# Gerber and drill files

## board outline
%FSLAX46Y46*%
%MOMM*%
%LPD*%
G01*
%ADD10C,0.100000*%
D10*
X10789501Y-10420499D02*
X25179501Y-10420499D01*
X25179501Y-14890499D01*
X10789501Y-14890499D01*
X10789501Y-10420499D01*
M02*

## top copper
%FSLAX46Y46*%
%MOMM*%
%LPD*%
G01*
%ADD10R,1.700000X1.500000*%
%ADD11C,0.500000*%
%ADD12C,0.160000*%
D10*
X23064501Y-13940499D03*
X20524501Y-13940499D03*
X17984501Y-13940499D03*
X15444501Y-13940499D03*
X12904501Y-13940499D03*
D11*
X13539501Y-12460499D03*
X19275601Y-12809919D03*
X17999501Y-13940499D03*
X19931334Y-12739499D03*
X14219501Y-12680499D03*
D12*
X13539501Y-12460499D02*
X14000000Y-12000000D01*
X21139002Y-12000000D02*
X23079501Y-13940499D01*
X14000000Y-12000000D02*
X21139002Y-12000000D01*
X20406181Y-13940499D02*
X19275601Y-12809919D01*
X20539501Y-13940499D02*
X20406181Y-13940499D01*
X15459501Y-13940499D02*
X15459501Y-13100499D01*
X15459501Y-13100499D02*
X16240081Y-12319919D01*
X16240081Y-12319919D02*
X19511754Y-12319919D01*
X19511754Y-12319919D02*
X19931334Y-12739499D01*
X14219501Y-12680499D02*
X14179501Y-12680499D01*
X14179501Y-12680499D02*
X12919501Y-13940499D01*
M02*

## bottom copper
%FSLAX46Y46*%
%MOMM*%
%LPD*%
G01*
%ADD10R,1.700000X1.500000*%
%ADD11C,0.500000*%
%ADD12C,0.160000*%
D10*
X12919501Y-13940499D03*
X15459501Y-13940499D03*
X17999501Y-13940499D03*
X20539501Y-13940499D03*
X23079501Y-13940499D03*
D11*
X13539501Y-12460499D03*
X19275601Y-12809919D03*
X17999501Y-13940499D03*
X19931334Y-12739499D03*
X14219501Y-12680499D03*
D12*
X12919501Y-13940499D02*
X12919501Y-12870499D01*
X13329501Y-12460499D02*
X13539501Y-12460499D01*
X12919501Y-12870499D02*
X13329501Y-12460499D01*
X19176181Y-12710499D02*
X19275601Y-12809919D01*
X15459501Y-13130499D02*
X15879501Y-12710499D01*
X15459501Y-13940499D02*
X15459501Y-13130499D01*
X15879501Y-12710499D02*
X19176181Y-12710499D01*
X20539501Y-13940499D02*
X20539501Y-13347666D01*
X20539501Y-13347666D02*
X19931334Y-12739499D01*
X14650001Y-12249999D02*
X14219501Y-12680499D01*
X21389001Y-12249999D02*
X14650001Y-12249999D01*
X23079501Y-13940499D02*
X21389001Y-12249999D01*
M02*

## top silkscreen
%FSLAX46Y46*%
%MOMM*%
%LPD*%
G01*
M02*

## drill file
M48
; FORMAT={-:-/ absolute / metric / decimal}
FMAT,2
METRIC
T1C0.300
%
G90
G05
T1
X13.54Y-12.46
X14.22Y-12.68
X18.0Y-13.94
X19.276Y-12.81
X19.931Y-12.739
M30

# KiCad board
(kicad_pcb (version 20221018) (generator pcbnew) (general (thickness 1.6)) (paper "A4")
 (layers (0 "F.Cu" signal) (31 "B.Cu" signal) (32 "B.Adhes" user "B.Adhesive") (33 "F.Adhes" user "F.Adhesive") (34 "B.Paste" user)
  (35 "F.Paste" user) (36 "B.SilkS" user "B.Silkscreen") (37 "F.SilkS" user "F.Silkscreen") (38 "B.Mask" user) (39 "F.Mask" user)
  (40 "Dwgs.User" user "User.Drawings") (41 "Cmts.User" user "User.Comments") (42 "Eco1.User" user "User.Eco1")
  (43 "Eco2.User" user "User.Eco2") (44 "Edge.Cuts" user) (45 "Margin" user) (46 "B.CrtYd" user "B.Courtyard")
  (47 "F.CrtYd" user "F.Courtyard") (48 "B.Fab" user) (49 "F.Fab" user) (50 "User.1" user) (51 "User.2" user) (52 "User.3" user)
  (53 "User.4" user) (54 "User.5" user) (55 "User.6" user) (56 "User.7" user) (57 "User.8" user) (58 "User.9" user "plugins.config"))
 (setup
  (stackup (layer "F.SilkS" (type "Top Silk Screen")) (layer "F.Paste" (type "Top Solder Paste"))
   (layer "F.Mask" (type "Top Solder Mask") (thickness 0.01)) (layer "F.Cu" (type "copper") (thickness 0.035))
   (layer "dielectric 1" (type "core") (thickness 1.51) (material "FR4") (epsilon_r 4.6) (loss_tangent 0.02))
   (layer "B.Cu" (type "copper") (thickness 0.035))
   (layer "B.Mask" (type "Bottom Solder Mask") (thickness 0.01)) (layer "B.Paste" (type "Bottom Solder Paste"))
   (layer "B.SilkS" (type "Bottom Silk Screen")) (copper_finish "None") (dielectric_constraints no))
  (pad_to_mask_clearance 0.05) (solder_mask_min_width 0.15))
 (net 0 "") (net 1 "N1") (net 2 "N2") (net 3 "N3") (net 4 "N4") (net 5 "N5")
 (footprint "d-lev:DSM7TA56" (layer "F.Cu") (at 17.984501 23.640499)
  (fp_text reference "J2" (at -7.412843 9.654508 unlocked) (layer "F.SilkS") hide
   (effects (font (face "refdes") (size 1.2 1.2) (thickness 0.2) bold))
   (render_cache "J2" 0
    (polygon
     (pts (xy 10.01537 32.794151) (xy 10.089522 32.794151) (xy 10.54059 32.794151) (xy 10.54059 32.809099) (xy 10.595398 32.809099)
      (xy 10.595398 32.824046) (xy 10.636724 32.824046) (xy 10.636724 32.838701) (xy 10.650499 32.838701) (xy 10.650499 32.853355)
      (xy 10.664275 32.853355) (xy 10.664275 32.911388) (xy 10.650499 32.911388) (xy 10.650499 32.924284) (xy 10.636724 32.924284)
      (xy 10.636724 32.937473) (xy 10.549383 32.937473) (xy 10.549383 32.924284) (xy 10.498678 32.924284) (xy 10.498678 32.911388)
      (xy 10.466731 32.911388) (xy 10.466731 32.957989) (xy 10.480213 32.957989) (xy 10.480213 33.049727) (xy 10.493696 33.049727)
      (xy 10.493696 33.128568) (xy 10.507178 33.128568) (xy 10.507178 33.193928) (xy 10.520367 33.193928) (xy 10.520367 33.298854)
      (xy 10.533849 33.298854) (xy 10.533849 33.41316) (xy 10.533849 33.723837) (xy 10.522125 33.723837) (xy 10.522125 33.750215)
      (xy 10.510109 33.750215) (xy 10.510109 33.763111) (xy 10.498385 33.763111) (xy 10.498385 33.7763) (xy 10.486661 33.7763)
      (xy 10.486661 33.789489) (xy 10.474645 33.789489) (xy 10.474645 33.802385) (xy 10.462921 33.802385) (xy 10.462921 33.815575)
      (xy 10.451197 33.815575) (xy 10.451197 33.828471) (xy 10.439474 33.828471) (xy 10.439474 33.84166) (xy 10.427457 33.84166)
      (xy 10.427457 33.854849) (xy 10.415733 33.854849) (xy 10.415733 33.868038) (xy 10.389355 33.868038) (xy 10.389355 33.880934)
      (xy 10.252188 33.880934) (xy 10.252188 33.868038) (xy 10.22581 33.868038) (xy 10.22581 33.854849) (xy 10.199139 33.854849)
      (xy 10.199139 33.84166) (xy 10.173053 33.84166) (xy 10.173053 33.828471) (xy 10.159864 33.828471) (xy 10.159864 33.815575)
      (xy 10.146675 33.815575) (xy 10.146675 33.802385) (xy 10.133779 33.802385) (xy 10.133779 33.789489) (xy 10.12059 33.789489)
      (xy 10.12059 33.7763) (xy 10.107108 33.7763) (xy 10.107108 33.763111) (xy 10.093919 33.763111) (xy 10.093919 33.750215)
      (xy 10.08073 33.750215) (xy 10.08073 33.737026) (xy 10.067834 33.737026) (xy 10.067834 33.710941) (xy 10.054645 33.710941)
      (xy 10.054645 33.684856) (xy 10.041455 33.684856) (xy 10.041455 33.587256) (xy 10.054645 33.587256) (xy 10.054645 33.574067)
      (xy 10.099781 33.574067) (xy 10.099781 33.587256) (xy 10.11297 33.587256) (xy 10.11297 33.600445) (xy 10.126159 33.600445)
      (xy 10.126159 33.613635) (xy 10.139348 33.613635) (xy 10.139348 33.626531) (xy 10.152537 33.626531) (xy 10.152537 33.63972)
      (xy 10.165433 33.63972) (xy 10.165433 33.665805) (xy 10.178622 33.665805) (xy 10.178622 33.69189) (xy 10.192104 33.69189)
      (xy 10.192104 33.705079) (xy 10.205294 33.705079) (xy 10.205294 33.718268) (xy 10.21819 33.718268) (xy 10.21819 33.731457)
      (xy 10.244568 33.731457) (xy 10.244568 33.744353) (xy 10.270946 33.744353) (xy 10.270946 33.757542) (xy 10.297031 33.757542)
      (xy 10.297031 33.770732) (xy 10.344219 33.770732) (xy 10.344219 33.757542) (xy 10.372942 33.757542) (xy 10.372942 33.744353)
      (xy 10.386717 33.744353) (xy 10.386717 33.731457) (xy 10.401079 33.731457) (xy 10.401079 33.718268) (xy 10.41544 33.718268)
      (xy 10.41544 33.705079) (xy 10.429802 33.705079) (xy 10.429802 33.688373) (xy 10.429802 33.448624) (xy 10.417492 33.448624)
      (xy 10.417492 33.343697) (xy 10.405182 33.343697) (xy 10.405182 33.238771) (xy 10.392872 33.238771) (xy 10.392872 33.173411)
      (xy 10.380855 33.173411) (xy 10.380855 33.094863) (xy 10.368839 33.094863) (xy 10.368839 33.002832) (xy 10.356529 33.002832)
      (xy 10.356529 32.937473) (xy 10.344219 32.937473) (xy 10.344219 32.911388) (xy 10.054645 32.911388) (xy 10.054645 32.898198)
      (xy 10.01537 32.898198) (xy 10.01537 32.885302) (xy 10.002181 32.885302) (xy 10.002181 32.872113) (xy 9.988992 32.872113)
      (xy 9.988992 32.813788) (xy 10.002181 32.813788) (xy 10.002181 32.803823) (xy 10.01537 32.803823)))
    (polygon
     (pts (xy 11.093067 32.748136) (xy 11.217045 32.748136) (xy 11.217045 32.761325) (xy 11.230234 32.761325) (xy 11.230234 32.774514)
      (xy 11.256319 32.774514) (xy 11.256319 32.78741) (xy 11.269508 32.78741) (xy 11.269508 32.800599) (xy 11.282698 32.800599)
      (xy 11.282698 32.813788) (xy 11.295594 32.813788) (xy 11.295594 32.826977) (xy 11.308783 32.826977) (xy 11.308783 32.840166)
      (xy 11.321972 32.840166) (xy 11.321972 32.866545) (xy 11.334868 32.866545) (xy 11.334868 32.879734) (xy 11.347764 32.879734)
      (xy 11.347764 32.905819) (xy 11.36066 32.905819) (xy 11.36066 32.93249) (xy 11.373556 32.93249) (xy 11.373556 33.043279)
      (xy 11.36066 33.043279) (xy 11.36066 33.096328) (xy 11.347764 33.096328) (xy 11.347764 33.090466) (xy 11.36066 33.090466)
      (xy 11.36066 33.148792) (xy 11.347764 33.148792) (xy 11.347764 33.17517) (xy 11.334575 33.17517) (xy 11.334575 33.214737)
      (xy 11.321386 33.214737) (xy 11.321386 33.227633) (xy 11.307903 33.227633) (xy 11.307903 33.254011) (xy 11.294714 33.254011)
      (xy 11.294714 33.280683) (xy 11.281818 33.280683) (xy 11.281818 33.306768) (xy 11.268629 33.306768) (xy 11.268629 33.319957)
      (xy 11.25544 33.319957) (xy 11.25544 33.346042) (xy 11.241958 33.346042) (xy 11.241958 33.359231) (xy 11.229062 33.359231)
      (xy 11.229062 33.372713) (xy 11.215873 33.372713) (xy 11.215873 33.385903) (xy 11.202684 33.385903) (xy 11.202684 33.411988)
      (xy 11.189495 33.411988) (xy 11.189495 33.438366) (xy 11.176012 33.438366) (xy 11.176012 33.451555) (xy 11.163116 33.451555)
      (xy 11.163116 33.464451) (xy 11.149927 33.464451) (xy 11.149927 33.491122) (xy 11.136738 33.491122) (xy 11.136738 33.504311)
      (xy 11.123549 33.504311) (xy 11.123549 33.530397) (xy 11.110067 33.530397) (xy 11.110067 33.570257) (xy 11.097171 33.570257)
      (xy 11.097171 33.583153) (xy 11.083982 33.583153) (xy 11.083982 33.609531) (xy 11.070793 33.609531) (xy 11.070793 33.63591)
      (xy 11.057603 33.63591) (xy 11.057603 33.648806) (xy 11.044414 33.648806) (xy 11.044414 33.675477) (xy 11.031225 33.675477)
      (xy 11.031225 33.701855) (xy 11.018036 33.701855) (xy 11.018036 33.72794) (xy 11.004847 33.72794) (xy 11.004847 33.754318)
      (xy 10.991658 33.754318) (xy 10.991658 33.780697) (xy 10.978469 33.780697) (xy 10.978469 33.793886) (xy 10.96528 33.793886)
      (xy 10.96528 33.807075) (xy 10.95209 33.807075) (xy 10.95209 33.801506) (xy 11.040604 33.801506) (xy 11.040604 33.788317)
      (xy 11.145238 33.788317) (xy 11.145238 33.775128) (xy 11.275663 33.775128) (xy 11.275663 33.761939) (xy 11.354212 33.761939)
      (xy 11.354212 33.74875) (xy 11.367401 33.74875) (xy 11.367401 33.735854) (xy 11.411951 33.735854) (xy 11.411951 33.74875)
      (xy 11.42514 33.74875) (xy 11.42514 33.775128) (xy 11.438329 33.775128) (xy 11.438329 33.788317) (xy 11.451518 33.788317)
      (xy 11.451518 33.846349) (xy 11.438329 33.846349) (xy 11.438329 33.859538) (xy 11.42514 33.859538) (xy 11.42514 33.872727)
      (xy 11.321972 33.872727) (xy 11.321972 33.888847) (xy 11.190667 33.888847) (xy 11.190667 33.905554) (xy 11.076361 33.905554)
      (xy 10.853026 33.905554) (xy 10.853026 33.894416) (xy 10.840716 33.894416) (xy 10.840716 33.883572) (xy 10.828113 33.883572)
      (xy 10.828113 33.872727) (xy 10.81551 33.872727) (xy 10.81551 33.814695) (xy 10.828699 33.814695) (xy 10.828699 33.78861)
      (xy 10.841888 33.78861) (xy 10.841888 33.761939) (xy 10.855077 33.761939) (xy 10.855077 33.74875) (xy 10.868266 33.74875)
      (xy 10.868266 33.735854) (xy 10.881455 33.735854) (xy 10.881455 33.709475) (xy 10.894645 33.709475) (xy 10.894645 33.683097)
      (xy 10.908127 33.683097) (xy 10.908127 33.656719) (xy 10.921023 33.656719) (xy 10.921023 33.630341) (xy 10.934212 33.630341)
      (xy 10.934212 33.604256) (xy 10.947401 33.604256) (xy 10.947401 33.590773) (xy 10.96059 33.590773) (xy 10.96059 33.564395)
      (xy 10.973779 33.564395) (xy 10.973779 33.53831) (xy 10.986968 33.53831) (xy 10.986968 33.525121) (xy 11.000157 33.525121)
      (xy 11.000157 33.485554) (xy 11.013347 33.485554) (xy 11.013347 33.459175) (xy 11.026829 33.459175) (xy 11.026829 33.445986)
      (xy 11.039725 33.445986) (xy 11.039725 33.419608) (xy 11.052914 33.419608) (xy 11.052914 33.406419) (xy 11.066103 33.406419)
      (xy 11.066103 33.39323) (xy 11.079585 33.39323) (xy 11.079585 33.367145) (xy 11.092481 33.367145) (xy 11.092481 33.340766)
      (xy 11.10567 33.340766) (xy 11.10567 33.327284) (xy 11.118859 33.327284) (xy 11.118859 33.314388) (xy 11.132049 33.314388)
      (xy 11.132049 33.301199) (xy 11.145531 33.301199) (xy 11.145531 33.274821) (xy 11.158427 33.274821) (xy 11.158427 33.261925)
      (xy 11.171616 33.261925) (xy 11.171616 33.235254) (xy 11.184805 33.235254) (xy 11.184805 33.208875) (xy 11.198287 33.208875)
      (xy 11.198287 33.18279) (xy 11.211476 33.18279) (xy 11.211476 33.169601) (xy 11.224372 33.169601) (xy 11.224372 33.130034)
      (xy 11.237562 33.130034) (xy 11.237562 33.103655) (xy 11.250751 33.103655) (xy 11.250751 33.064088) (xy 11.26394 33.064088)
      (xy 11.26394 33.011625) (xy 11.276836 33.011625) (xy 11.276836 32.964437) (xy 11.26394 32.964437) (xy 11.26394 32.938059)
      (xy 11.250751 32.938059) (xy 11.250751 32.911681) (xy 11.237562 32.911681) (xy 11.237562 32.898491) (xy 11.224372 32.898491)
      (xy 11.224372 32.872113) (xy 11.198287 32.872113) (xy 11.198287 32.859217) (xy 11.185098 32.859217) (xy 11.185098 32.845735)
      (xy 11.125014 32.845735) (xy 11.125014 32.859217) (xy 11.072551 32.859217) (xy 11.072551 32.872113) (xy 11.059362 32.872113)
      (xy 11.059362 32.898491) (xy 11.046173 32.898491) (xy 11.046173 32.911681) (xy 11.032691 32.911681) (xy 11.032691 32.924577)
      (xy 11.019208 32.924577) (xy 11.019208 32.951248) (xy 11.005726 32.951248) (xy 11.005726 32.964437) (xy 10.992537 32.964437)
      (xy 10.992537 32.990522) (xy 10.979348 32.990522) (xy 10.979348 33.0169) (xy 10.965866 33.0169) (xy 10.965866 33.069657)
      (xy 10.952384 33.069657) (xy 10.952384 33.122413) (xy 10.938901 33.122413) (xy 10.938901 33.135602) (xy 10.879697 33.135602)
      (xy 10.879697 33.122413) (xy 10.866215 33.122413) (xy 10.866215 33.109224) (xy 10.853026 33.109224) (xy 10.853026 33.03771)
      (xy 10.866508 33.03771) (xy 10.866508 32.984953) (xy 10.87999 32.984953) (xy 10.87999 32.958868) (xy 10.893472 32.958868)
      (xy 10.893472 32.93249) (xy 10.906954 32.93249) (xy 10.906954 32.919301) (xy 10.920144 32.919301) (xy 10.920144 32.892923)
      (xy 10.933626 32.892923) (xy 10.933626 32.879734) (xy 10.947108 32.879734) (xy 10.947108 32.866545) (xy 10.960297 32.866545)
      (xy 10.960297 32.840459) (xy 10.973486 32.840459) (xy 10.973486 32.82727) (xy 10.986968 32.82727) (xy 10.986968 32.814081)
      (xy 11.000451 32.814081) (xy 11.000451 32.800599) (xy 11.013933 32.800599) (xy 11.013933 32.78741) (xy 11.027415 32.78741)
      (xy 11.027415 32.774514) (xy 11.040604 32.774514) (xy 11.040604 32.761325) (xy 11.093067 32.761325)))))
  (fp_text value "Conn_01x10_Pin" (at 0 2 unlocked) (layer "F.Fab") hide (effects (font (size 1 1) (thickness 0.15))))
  (pad "6" smd rect (at 5.08 -9.7) (size 1.7 1.5) (layers "F.Cu" "F.Paste" "F.Mask") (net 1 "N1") (thermal_bridge_angle 45))
  (pad "7" smd rect (at 2.54 -9.7) (size 1.7 1.5) (layers "F.Cu" "F.Paste" "F.Mask") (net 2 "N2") (thermal_bridge_angle 45))
  (pad "8" smd rect (at 0 -9.7) (size 1.7 1.5) (layers "F.Cu" "F.Paste" "F.Mask") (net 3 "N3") (thermal_bridge_angle 45))
  (pad "9" smd rect (at -2.54 -9.7) (size 1.7 1.5) (layers "F.Cu" "F.Paste" "F.Mask") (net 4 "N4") (thermal_bridge_angle 45))
  (pad "10" smd rect (at -5.08 -9.7) (size 1.7 1.5) (layers "F.Cu" "F.Paste" "F.Mask") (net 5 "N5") (thermal_bridge_angle 45)))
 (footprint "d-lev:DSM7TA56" (layer "B.Cu") (at 17.999501 23.640499 180)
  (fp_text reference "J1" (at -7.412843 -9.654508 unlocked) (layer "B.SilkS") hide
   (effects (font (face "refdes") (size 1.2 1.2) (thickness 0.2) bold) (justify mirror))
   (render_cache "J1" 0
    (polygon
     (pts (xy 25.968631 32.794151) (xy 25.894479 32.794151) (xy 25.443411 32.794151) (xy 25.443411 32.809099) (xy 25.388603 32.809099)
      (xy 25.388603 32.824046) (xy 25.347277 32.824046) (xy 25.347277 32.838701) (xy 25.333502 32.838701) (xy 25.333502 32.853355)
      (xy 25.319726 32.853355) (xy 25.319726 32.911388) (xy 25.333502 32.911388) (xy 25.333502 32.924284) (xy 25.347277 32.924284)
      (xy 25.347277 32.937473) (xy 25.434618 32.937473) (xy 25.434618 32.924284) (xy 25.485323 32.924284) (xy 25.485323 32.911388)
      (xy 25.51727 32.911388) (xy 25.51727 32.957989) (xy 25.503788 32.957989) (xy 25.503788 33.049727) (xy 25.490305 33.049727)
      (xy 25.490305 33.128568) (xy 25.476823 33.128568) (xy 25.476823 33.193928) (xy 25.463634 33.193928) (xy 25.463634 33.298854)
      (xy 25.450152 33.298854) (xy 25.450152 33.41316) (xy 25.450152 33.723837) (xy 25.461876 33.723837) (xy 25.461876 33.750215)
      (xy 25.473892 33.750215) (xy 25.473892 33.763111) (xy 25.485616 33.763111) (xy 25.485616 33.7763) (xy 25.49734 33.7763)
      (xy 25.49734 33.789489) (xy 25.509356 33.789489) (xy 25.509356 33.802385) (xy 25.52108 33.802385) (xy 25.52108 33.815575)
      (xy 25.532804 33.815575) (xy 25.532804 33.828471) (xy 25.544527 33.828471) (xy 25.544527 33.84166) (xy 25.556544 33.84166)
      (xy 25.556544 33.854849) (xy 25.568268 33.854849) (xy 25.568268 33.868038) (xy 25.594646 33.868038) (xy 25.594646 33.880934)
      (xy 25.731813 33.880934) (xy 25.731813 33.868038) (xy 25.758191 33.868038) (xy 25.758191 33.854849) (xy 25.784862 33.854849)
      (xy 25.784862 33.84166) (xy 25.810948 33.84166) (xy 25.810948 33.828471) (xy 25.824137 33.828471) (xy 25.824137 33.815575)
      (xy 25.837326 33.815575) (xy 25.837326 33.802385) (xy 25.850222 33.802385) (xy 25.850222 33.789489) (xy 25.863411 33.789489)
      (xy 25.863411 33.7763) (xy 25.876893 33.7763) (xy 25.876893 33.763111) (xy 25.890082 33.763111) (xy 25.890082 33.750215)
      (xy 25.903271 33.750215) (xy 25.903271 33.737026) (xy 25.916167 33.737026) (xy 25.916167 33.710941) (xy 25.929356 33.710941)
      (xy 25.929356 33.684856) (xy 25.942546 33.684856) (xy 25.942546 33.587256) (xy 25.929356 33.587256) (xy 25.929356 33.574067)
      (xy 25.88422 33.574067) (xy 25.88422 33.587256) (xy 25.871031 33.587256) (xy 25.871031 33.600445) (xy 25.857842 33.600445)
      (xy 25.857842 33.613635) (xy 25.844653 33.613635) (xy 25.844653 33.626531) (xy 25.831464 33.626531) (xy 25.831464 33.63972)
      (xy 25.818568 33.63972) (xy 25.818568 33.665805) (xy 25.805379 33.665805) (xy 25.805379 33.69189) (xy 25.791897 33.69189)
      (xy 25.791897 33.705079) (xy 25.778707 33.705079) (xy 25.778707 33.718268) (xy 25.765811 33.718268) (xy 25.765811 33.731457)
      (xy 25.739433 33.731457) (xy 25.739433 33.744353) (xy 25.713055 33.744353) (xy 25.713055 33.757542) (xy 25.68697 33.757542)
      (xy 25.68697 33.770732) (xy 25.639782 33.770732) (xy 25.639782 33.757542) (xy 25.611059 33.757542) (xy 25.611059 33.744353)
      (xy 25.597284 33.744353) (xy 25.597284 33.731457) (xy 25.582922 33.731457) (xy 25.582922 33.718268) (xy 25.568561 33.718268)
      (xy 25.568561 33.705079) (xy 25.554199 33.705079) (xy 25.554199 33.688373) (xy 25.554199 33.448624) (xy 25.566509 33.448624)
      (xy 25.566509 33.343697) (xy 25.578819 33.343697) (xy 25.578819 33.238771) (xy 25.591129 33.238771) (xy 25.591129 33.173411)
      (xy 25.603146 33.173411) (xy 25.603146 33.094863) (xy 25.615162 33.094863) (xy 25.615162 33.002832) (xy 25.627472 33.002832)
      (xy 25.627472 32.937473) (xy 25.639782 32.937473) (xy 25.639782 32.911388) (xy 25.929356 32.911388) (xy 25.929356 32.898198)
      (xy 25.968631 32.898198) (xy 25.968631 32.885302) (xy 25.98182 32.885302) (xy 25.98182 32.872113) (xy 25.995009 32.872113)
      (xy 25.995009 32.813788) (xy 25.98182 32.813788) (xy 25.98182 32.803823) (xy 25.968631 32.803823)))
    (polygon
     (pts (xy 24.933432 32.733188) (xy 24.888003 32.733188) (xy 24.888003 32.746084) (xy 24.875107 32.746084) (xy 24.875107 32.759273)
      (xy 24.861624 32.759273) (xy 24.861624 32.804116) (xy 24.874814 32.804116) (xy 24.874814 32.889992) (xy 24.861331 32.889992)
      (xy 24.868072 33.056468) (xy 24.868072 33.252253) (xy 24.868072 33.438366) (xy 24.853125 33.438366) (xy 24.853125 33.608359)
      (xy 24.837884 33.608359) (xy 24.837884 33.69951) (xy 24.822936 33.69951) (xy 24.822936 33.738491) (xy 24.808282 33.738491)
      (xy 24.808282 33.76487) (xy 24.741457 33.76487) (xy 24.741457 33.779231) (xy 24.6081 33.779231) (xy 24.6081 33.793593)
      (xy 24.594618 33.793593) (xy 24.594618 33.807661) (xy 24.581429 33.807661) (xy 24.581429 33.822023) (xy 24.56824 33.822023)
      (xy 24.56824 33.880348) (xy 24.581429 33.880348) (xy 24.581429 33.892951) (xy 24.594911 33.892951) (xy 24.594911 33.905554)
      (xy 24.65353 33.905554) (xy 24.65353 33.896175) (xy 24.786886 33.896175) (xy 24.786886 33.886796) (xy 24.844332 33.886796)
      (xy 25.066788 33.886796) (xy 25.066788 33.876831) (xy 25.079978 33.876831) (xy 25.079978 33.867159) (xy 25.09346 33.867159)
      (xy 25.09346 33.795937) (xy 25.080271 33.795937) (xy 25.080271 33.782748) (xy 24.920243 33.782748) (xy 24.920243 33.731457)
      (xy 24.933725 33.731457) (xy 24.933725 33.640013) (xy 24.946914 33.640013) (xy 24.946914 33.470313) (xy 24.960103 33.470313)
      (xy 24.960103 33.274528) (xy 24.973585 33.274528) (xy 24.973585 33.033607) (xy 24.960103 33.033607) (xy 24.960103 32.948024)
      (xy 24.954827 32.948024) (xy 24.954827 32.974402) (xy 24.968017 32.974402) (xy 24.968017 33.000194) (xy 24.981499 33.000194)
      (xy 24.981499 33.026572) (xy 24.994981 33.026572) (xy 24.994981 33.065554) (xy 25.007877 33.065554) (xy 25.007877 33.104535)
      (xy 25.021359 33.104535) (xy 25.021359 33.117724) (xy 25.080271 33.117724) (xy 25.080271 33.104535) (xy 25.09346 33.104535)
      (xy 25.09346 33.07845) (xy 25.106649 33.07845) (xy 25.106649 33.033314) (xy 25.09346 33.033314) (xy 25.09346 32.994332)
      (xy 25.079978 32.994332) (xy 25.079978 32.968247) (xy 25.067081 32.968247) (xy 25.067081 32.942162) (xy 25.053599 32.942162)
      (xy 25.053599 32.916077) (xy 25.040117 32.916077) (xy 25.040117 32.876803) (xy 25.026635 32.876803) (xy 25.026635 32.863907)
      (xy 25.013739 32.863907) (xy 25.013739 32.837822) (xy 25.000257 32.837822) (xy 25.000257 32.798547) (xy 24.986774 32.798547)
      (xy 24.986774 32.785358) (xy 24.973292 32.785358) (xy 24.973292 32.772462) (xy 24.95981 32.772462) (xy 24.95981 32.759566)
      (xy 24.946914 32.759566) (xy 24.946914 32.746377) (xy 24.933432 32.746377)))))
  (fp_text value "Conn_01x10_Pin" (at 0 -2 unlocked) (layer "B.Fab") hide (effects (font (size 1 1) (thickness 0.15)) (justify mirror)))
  (pad "6" smd rect (at 5.08 9.7 180) (size 1.7 1.5) (layers "B.Cu" "B.Paste" "B.Mask") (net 1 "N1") (thermal_bridge_angle 45))
  (pad "7" smd rect (at 2.54 9.7 180) (size 1.7 1.5) (layers "B.Cu" "B.Paste" "B.Mask") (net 2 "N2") (thermal_bridge_angle 45))
  (pad "8" smd rect (at 0 9.7 180) (size 1.7 1.5) (layers "B.Cu" "B.Paste" "B.Mask") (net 3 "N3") (thermal_bridge_angle 45))
  (pad "9" smd rect (at -2.54 9.7 180) (size 1.7 1.5) (layers "B.Cu" "B.Paste" "B.Mask") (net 4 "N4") (thermal_bridge_angle 45))
  (pad "10" smd rect (at -5.08 9.7 180) (size 1.7 1.5) (layers "B.Cu" "B.Paste" "B.Mask") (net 5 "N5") (thermal_bridge_angle 45)))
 (gr_rect (start 10.789501 10.420499) (end 25.179501 14.890499) (stroke (width 0.1) (type default)) (fill none) (layer "Edge.Cuts"))
 (segment (start 13.539501 12.460499) (end 14 12) (width 0.16) (layer "F.Cu") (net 1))
 (segment (start 21.139002 12) (end 23.079501 13.940499) (width 0.16) (layer "F.Cu") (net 1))
 (segment (start 14 12) (end 21.139002 12) (width 0.16) (layer "F.Cu") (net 1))
 (via (at 13.539501 12.460499) (size 0.5) (drill 0.3) (layers "F.Cu" "B.Cu") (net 1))
 (segment (start 12.919501 13.940499) (end 12.919501 12.870499) (width 0.16) (layer "B.Cu") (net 1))
 (segment (start 13.329501 12.460499) (end 13.539501 12.460499) (width 0.16) (layer "B.Cu") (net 1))
 (segment (start 12.919501 12.870499) (end 13.329501 12.460499) (width 0.16) (layer "B.Cu") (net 1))
 (segment (start 20.406181 13.940499) (end 19.275601 12.809919) (width 0.16) (layer "F.Cu") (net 2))
 (segment (start 20.539501 13.940499) (end 20.406181 13.940499) (width 0.16) (layer "F.Cu") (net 2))
 (via (at 19.275601 12.809919) (size 0.5) (drill 0.3) (layers "F.Cu" "B.Cu") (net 2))
 (segment (start 19.176181 12.710499) (end 19.275601 12.809919) (width 0.16) (layer "B.Cu") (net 2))
 (segment (start 15.459501 13.130499) (end 15.879501 12.710499) (width 0.16) (layer "B.Cu") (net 2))
 (segment (start 15.459501 13.940499) (end 15.459501 13.130499) (width 0.16) (layer "B.Cu") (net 2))
 (segment (start 15.879501 12.710499) (end 19.176181 12.710499) (width 0.16) (layer "B.Cu") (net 2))
 (via (at 17.999501 13.940499) (size 0.5) (drill 0.3) (layers "F.Cu" "B.Cu") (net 3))
 (segment (start 15.459501 13.940499) (end 15.459501 13.100499) (width 0.16) (layer "F.Cu") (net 4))
 (segment (start 15.459501 13.100499) (end 16.240081 12.319919) (width 0.16) (layer "F.Cu") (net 4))
 (segment (start 16.240081 12.319919) (end 19.511754 12.319919) (width 0.16) (layer "F.Cu") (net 4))
 (segment (start 19.511754 12.319919) (end 19.931334 12.739499) (width 0.16) (layer "F.Cu") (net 4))
 (via (at 19.931334 12.739499) (size 0.5) (drill 0.3) (layers "F.Cu" "B.Cu") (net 4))
 (segment (start 20.539501 13.940499) (end 20.539501 13.347666) (width 0.16) (layer "B.Cu") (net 4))
 (segment (start 20.539501 13.347666) (end 19.931334 12.739499) (width 0.16) (layer "B.Cu") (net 4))
 (segment (start 14.219501 12.680499) (end 14.179501 12.680499) (width 0.16) (layer "F.Cu") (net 5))
 (segment (start 14.179501 12.680499) (end 12.919501 13.940499) (width 0.16) (layer "F.Cu") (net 5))
 (via (at 14.219501 12.680499) (size 0.5) (drill 0.3) (layers "F.Cu" "B.Cu") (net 5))
 (segment (start 14.650001 12.249999) (end 14.219501 12.680499) (width 0.16) (layer "B.Cu") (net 5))
 (segment (start 21.389001 12.249999) (end 14.650001 12.249999) (width 0.16) (layer "B.Cu") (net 5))
 (segment (start 23.079501 13.940499) (end 21.389001 12.249999) (width 0.16) (layer "B.Cu") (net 5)))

